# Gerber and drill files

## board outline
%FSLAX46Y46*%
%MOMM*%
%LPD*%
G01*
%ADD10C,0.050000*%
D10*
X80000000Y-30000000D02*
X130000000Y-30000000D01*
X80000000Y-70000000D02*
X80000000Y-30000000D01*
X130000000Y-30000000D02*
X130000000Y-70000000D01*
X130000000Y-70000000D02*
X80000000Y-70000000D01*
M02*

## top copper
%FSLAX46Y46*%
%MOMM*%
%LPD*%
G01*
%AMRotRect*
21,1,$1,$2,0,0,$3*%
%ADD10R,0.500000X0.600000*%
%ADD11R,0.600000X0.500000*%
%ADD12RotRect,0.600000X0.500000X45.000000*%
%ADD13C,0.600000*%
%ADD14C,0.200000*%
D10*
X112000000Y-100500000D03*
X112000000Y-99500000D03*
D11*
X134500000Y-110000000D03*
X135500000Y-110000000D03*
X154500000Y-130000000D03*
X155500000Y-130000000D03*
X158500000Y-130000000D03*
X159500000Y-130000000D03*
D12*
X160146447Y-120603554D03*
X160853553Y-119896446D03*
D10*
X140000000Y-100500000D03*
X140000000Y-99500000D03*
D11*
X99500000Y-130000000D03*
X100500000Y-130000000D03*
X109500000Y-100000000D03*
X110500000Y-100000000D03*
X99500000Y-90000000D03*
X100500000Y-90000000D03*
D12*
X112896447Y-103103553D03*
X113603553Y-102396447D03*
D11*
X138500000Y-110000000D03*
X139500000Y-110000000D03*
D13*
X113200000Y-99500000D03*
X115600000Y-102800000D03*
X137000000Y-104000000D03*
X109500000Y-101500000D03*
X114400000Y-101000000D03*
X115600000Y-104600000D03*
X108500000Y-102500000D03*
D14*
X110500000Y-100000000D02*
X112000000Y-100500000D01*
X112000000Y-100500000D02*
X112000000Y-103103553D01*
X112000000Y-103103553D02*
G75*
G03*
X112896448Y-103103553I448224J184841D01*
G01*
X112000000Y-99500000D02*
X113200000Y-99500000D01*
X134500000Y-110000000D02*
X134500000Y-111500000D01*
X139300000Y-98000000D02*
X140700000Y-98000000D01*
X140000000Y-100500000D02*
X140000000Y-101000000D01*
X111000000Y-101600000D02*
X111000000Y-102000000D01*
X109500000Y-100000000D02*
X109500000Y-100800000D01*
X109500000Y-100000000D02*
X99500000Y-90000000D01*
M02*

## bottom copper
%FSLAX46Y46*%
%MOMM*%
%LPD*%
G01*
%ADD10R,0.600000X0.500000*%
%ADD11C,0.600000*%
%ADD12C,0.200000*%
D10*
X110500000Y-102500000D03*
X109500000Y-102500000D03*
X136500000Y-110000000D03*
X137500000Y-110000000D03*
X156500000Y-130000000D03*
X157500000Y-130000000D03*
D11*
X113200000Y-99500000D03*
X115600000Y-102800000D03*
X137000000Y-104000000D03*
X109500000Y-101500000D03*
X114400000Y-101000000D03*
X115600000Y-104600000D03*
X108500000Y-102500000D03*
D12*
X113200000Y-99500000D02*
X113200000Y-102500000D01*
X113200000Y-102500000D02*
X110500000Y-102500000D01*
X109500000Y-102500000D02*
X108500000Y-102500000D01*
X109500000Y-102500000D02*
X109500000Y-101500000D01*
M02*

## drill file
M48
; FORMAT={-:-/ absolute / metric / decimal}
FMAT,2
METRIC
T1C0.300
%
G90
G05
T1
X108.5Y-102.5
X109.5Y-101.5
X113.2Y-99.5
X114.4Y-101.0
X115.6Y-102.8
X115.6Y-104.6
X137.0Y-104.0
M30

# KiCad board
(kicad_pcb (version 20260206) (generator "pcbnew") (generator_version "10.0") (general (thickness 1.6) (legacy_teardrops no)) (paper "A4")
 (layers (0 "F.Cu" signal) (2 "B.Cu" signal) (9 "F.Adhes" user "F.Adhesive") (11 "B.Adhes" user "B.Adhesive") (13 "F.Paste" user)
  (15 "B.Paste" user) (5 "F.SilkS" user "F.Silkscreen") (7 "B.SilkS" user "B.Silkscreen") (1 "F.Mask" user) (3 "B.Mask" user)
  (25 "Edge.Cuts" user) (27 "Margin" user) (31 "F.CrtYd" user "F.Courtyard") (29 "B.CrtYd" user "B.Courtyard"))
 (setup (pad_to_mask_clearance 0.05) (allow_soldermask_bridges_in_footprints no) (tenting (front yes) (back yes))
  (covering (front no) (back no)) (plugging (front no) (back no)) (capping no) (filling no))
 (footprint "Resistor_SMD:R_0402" (layer "F.Cu") (at 112 100 90)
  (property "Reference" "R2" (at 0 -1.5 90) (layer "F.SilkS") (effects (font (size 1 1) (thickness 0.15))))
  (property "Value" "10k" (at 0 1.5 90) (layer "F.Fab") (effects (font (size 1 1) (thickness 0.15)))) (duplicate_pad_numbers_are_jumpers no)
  (pad "1" smd rect (at -0.5 0 90) (size 0.6 0.5) (layers "F.Cu" "F.Mask" "F.Paste") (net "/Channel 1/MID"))
  (pad "2" smd rect (at 0.5 0 90) (size 0.6 0.5) (layers "F.Cu" "F.Mask" "F.Paste") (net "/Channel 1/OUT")))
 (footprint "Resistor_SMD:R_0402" (layer "F.Cu") (at 135 110)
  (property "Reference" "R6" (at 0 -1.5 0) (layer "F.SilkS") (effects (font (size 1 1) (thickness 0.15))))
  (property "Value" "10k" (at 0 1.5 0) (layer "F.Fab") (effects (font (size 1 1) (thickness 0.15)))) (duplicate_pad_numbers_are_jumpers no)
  (pad "1" smd rect (at -0.5 0) (size 0.6 0.5) (layers "F.Cu" "F.Mask" "F.Paste") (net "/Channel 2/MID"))
  (pad "2" smd rect (at 0.5 0) (size 0.6 0.5) (layers "F.Cu" "F.Mask" "F.Paste") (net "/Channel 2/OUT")))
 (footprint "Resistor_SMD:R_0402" (layer "F.Cu") (at 155 130)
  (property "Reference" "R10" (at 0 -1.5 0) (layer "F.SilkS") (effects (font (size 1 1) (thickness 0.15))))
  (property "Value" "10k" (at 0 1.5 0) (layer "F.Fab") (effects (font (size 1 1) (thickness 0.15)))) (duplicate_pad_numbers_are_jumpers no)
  (pad "1" smd rect (at -0.5 0) (size 0.6 0.5) (layers "F.Cu" "F.Mask" "F.Paste") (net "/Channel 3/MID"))
  (pad "2" smd rect (at 0.5 0) (size 0.6 0.5) (layers "F.Cu" "F.Mask" "F.Paste") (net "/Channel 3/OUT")))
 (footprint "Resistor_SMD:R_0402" (layer "F.Cu") (at 159 130)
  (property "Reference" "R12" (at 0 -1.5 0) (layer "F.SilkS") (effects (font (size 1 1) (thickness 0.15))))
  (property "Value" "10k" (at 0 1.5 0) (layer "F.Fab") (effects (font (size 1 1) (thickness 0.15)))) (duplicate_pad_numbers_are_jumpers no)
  (pad "1" smd rect (at -0.5 0) (size 0.6 0.5) (layers "F.Cu" "F.Mask" "F.Paste") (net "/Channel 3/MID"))
  (pad "2" smd rect (at 0.5 0) (size 0.6 0.5) (layers "F.Cu" "F.Mask" "F.Paste") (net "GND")))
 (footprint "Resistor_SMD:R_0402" (layer "F.Cu") (at 160.5 120.25 45)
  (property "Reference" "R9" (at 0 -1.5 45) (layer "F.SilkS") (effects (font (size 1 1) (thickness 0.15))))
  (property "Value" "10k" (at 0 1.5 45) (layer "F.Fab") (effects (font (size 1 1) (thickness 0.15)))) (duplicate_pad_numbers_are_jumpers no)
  (pad "1" smd rect (at -0.5 0.000001 45) (size 0.6 0.5) (layers "F.Cu" "F.Mask" "F.Paste") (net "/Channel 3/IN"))
  (pad "2" smd rect (at 0.5 -0.000001 45) (size 0.6 0.5) (layers "F.Cu" "F.Mask" "F.Paste") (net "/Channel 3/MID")))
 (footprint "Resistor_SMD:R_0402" (layer "F.Cu") (at 140 100 90)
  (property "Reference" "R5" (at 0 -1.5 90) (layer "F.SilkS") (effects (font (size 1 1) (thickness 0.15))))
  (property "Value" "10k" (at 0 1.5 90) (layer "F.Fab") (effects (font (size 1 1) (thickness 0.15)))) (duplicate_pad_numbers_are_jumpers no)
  (pad "1" smd rect (at -0.5 0 90) (size 0.6 0.5) (layers "F.Cu" "F.Mask" "F.Paste") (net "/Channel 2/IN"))
  (pad "2" smd rect (at 0.5 0 90) (size 0.6 0.5) (layers "F.Cu" "F.Mask" "F.Paste") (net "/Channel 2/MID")))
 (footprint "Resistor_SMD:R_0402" (layer "F.Cu") (at 100 130)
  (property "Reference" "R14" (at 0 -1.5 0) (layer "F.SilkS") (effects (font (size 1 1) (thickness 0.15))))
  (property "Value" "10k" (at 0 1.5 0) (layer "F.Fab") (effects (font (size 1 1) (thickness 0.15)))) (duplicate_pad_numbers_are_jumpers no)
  (pad "1" smd rect (at -0.5 0) (size 0.6 0.5) (layers "F.Cu" "F.Mask" "F.Paste") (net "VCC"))
  (pad "2" smd rect (at 0.5 0) (size 0.6 0.5) (layers "F.Cu" "F.Mask" "F.Paste") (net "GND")))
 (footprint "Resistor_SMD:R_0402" (layer "F.Cu") (at 110 100)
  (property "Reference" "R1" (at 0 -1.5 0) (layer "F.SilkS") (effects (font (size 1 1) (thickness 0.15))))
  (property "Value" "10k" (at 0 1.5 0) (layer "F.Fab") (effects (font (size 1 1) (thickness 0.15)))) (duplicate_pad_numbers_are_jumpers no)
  (pad "1" smd rect (at -0.5 0) (size 0.6 0.5) (layers "F.Cu" "F.Mask" "F.Paste") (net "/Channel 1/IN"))
  (pad "2" smd rect (at 0.5 0) (size 0.6 0.5) (layers "F.Cu" "F.Mask" "F.Paste") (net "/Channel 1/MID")))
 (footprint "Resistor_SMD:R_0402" (layer "F.Cu") (at 100 90)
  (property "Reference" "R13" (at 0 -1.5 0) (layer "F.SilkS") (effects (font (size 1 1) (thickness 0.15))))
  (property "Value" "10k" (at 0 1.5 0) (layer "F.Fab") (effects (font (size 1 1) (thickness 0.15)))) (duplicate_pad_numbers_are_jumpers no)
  (pad "1" smd rect (at -0.5 0) (size 0.6 0.5) (layers "F.Cu" "F.Mask" "F.Paste") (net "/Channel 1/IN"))
  (pad "2" smd rect (at 0.5 0) (size 0.6 0.5) (layers "F.Cu" "F.Mask" "F.Paste") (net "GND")))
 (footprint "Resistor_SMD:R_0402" (layer "F.Cu") (at 113.25 102.75 45)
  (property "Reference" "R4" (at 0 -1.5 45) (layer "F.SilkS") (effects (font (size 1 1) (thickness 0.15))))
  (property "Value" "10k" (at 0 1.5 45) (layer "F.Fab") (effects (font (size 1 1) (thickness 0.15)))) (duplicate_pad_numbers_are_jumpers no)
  (pad "1" smd rect (at -0.499999 0 45) (size 0.6 0.5) (layers "F.Cu" "F.Mask" "F.Paste") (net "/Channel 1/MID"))
  (pad "2" smd rect (at 0.499999 0 45) (size 0.6 0.5) (layers "F.Cu" "F.Mask" "F.Paste") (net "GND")))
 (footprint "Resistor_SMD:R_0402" (layer "F.Cu") (at 139 110)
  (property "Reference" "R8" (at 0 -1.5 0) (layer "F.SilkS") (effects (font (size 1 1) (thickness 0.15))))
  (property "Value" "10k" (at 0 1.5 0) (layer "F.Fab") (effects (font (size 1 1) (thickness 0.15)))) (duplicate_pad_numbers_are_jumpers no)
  (pad "1" smd rect (at -0.5 0) (size 0.6 0.5) (layers "F.Cu" "F.Mask" "F.Paste") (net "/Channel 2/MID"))
  (pad "2" smd rect (at 0.5 0) (size 0.6 0.5) (layers "F.Cu" "F.Mask" "F.Paste") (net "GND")))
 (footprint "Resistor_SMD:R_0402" (layer "B.Cu") (at 110 102.5 180)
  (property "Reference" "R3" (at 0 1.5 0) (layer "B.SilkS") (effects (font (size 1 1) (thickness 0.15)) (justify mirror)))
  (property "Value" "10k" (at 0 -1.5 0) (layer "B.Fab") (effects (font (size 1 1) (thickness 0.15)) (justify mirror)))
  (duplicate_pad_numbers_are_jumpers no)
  (pad "1" smd rect (at -0.5 0 180) (size 0.6 0.5) (layers "B.Cu" "B.Mask" "B.Paste") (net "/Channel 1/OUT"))
  (pad "2" smd rect (at 0.5 0 180) (size 0.6 0.5) (layers "B.Cu" "B.Mask" "B.Paste") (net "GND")))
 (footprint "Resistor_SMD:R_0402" (layer "B.Cu") (at 137 110)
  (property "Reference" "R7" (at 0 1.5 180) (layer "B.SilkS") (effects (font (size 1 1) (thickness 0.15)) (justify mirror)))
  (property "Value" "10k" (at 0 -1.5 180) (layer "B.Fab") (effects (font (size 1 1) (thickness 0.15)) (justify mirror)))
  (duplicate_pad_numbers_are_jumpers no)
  (pad "1" smd rect (at -0.5 0) (size 0.6 0.5) (layers "B.Cu" "B.Mask" "B.Paste") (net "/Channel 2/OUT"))
  (pad "2" smd rect (at 0.5 0) (size 0.6 0.5) (layers "B.Cu" "B.Mask" "B.Paste") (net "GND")))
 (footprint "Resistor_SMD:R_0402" (layer "B.Cu") (at 157 130)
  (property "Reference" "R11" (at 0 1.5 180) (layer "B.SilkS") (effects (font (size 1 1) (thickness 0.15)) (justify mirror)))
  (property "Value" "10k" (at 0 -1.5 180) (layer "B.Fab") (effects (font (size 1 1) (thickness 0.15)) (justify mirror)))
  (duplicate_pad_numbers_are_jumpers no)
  (pad "1" smd rect (at -0.5 0) (size 0.6 0.5) (layers "B.Cu" "B.Mask" "B.Paste") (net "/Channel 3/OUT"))
  (pad "2" smd rect (at 0.5 0) (size 0.6 0.5) (layers "B.Cu" "B.Mask" "B.Paste") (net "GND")))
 (gr_line (start 80 30) (end 130 30) (stroke (width 0.05) (type default)) (layer "Edge.Cuts"))
 (gr_line (start 80 70) (end 80 30) (stroke (width 0.05) (type default)) (layer "Edge.Cuts"))
 (gr_line (start 130 30) (end 130 70) (stroke (width 0.05) (type default)) (layer "Edge.Cuts"))
 (gr_line (start 130 70) (end 80 70) (stroke (width 0.05) (type default)) (layer "Edge.Cuts"))
 (segment (start 110.5 100) (end 112 100.5) (width 0.2) (locked yes) (layer "F.Cu") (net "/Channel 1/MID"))
 (segment (start 112 100.5) (end 112 103.103553) (width 0.2) (layer "F.Cu") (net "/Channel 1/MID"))
 (arc (start 112 103.103553) (mid 112.448223 103.403553) (end 112.896447 103.103553) (width 0.2) (layer "F.Cu") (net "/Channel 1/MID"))
 (segment (start 112 99.5) (end 113.2 99.5) (width 0.2) (layer "F.Cu") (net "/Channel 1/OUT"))
 (via (at 113.2 99.5) (size 0.6) (drill 0.3) (layers "F.Cu" "B.Cu") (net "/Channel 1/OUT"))
 (segment (start 113.2 99.5) (end 113.2 102.5) (width 0.2) (layer "B.Cu") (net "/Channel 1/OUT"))
 (segment (start 113.2 102.5) (end 110.5 102.5) (width 0.2) (layer "B.Cu") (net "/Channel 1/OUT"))
 (segment (start 134.5 110) (end 134.5 111.5) (width 0.2) (layer "F.Cu") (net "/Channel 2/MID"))
 (segment (start 139.3 98) (end 140.7 98) (width 0.2) (layer "F.Cu") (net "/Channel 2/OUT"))
 (via (at 115.6 102.8) (size 0.6) (drill 0.3) (layers "F.Cu" "B.Cu") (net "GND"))
 (via (at 137 104) (size 0.6) (drill 0.3) (layers "F.Cu" "B.Cu") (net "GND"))
 (via (at 109.5 101.5) (size 0.6) (drill 0.3) (layers "F.Cu" "B.Cu") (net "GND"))
 (via (at 114.4 101) (size 0.6) (drill 0.3) (layers "F.Cu" "B.Cu") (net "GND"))
 (via (at 115.6 104.6) (size 0.6) (drill 0.3) (layers "F.Cu" "B.Cu") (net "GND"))
 (via (at 108.5 102.5) (size 0.6) (drill 0.3) (layers "F.Cu" "B.Cu") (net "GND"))
 (segment (start 109.5 102.5) (end 108.5 102.5) (width 0.2) (layer "B.Cu") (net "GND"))
 (segment (start 109.5 102.5) (end 109.5 101.5) (width 0.2) (layer "B.Cu") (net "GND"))
 (segment (start 140 100.5) (end 140 101) (width 0.2) (layer "F.Cu") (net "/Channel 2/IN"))
 (segment (start 111 101.6) (end 111 102) (width 0.2) (layer "F.Cu") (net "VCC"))
 (segment (start 109.5 100) (end 109.5 100.8) (width 0.2) (layer "F.Cu") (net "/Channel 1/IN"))
 (segment (start 109.5 100) (end 99.5 90) (width 0.2) (layer "F.Cu") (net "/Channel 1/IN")))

